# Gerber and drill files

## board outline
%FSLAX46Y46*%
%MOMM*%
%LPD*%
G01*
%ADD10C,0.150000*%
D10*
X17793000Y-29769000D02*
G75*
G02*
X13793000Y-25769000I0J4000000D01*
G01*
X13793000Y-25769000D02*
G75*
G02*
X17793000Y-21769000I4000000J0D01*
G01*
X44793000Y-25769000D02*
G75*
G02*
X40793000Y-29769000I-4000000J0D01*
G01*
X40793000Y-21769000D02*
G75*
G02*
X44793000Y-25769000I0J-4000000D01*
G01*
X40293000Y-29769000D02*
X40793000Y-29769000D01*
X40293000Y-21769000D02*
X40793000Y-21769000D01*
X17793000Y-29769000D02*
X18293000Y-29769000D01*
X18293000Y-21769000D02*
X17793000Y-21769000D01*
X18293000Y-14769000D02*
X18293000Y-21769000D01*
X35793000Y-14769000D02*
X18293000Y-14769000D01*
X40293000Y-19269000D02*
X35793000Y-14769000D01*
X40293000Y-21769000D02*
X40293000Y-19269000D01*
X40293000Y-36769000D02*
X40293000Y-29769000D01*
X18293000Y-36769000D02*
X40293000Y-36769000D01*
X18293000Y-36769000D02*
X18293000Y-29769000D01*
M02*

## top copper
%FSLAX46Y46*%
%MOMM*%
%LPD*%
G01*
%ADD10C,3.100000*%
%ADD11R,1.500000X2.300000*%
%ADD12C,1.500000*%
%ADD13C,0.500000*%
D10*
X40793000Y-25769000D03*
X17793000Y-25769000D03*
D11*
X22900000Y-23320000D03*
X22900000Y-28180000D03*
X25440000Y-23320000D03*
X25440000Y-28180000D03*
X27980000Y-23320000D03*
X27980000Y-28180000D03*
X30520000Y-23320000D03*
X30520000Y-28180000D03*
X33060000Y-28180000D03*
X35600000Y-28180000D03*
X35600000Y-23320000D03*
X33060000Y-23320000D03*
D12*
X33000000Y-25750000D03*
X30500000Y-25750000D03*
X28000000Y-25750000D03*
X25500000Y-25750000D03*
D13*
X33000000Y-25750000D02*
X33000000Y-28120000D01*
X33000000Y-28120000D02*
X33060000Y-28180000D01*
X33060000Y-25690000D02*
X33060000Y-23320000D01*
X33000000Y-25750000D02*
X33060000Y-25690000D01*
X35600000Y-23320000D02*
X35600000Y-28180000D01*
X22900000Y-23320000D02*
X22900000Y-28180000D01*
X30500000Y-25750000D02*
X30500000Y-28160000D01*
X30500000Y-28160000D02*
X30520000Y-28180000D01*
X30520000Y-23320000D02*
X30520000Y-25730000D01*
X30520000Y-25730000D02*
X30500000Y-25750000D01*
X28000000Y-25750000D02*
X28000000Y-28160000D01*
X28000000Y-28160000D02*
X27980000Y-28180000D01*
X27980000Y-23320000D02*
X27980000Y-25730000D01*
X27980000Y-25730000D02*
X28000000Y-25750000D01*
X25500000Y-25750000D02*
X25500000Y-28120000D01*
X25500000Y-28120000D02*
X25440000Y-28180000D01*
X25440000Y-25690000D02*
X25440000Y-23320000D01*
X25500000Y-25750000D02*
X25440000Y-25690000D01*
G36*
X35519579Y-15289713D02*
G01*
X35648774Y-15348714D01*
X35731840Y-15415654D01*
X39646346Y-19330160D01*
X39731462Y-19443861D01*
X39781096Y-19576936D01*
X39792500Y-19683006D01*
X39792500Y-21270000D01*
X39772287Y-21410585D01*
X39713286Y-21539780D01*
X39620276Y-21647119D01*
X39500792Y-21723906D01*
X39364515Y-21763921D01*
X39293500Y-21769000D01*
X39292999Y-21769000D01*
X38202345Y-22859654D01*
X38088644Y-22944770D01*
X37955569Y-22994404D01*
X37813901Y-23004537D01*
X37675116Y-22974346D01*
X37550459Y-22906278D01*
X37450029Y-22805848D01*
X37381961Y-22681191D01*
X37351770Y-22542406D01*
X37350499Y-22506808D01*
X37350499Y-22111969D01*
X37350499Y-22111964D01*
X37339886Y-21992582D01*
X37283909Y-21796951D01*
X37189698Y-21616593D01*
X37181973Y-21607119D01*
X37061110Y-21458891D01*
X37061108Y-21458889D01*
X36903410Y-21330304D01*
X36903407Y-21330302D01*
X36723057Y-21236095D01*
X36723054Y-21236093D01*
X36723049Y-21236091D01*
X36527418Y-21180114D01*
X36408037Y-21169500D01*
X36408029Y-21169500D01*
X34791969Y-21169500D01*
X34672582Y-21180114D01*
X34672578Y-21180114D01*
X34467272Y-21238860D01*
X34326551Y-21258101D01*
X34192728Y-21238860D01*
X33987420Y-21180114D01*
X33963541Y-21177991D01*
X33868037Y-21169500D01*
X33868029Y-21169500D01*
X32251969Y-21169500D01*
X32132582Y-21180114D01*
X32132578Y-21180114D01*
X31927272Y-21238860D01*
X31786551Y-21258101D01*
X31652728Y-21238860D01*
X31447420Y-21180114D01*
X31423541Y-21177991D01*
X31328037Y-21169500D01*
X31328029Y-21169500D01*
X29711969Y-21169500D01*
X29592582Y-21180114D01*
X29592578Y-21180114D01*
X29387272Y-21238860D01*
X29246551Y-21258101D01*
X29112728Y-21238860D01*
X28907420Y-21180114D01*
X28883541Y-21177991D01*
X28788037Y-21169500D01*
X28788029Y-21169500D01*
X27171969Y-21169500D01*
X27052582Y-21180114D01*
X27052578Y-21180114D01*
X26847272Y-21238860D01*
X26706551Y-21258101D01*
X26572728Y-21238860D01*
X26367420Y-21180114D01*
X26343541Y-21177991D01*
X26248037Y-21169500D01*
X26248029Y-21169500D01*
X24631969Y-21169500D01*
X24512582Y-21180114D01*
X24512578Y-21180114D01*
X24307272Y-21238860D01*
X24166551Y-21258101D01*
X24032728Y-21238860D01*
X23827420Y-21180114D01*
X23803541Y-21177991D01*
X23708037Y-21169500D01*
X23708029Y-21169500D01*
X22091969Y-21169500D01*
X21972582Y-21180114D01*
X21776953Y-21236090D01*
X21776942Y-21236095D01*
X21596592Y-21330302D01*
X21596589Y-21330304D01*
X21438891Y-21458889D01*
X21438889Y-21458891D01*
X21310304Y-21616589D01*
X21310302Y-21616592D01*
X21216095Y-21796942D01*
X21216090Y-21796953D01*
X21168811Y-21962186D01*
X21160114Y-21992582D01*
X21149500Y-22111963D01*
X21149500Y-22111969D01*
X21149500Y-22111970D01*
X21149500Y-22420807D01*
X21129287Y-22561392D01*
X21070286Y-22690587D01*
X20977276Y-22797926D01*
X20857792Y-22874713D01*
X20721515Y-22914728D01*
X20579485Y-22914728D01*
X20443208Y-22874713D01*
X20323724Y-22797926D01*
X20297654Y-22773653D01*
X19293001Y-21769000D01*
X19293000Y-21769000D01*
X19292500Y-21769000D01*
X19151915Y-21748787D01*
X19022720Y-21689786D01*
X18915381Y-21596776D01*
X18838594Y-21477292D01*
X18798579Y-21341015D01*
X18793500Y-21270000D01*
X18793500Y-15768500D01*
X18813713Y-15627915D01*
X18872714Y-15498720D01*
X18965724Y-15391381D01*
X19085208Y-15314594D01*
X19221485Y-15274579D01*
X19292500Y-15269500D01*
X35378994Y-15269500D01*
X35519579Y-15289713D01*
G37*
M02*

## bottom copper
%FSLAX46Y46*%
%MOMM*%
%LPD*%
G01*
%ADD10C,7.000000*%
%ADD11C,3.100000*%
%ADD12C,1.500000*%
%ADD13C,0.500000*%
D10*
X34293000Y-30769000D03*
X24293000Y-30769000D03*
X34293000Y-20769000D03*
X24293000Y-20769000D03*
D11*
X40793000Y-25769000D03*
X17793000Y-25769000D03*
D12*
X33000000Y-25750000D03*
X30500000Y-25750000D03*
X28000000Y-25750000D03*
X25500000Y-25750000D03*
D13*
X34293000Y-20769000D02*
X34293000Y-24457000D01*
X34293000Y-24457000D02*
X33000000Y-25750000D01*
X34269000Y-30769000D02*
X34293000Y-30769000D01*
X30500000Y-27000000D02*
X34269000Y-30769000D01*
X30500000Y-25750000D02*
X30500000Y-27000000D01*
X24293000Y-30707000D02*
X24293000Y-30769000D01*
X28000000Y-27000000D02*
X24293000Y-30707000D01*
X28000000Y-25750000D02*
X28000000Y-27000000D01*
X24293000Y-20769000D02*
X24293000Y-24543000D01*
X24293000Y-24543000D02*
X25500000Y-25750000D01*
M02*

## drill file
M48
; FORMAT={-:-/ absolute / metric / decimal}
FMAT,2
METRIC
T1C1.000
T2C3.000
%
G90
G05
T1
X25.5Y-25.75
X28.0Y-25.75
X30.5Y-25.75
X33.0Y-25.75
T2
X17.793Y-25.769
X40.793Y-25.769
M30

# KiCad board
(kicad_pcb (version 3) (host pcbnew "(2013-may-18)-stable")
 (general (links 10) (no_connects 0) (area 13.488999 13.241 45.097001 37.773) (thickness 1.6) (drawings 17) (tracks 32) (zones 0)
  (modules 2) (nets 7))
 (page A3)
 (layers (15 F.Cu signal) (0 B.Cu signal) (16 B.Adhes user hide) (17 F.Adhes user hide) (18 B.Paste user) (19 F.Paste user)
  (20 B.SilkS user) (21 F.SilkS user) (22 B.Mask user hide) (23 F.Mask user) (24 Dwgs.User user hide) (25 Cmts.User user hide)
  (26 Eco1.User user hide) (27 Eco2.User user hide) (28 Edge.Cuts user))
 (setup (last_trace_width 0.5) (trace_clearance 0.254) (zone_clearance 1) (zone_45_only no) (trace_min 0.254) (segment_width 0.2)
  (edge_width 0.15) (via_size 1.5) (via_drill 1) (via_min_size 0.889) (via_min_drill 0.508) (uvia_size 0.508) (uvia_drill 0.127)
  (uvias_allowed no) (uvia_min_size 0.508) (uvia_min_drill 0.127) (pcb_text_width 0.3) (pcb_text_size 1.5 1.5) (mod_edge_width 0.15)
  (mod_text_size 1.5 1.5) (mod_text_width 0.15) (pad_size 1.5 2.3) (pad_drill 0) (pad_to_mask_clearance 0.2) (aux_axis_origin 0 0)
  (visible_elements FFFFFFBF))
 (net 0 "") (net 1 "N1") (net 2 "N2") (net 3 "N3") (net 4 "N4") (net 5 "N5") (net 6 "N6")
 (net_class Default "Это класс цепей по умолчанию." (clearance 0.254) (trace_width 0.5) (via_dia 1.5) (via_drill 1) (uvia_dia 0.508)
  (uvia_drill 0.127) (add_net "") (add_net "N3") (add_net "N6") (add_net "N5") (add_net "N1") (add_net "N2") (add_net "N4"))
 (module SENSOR (layer B.Cu) (at 40.793 37.269 180)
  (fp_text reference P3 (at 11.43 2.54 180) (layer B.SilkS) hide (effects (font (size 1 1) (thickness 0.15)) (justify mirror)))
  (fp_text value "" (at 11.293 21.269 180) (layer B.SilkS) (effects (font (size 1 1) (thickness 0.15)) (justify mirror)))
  (pad 2 smd circle (at 6.5 6.5 180) (size 7 7) (layers B.Cu B.Mask) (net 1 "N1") (solder_mask_margin 0.1))
  (pad 3 smd circle (at 16.5 6.5 180) (size 7 7) (layers B.Cu B.Mask) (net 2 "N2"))
  (pad 1 smd circle (at 6.5 16.5 180) (size 7 7) (layers B.Cu B.Mask) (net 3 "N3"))
  (pad 4 smd circle (at 16.5 16.5 180) (size 7 7) (layers B.Cu B.Mask) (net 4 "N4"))
  (pad "" np_thru_hole circle (at 0 11.5 180) (size 3.1 3.1) (drill 3) (layers *.Cu *.Mask B.SilkS))
  (pad "" np_thru_hole circle (at 23 11.5 180) (size 3.1 3.1) (drill 3) (layers *.Cu *.Mask B.SilkS)))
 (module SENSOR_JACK (layer F.Cu) (at 29.25 25.75)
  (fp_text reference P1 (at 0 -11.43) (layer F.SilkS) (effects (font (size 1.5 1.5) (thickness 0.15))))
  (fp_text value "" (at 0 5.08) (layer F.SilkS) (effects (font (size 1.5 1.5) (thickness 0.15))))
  (pad 12 smd rect (at -6.35 -2.43) (size 1.5 2.3) (layers F.Cu F.Paste F.Mask) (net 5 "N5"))
  (pad 1 smd rect (at -6.35 2.43) (size 1.5 2.3) (layers F.Cu F.Paste F.Mask) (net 5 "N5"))
  (pad 11 smd rect (at -3.81 -2.43) (size 1.5 2.3) (layers F.Cu F.Paste F.Mask) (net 4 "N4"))
  (pad 2 smd rect (at -3.81 2.43) (size 1.5 2.3) (layers F.Cu F.Paste F.Mask) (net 4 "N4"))
  (pad 10 smd rect (at -1.27 -2.43) (size 1.5 2.3) (layers F.Cu F.Paste F.Mask) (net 2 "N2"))
  (pad 3 smd rect (at -1.27 2.43) (size 1.5 2.3) (layers F.Cu F.Paste F.Mask) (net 2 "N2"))
  (pad 9 smd rect (at 1.27 -2.43) (size 1.5 2.3) (layers F.Cu F.Paste F.Mask) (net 1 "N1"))
  (pad 4 smd rect (at 1.27 2.43) (size 1.5 2.3) (layers F.Cu F.Paste F.Mask) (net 1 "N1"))
  (pad 5 smd rect (at 3.81 2.43) (size 1.5 2.3) (layers F.Cu F.Paste F.Mask) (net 3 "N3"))
  (pad 6 smd rect (at 6.35 2.43) (size 1.5 2.3) (layers F.Cu F.Paste F.Mask) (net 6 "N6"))
  (pad 7 smd rect (at 6.35 -2.43) (size 1.5 2.3) (layers F.Cu F.Paste F.Mask) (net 6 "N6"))
  (pad 8 smd rect (at 3.81 -2.43) (size 1.5 2.3) (layers F.Cu F.Paste F.Mask) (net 3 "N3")))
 (gr_arc (start 17.793 25.769) (end 17.793 29.769) (angle 90) (layer Edge.Cuts) (width 0.15))
 (gr_arc (start 17.793 25.769) (end 13.793 25.769) (angle 90) (layer Edge.Cuts) (width 0.15))
 (gr_arc (start 40.793 25.769) (end 44.793 25.769) (angle 90) (layer Edge.Cuts) (width 0.15))
 (gr_arc (start 40.793 25.769) (end 40.793 21.769) (angle 90) (layer Edge.Cuts) (width 0.15))
 (gr_line (start 40.293 29.769) (end 40.793 29.769) (angle 90) (layer Edge.Cuts) (width 0.15))
 (gr_line (start 40.293 21.769) (end 40.793 21.769) (angle 90) (layer Edge.Cuts) (width 0.15))
 (gr_line (start 17.793 29.769) (end 18.293 29.769) (angle 90) (layer Edge.Cuts) (width 0.15))
 (gr_line (start 18.293 21.769) (end 17.793 21.769) (angle 90) (layer Edge.Cuts) (width 0.15))
 (gr_line (start 18.293 14.769) (end 18.293 21.769) (angle 90) (layer Edge.Cuts) (width 0.15))
 (gr_line (start 35.793 14.769) (end 18.293 14.769) (angle 90) (layer Edge.Cuts) (width 0.15))
 (gr_line (start 40.293 19.269) (end 35.793 14.769) (angle 90) (layer Edge.Cuts) (width 0.15))
 (gr_line (start 40.293 21.769) (end 40.293 19.269) (angle 90) (layer Edge.Cuts) (width 0.15))
 (gr_line (start 40.293 36.769) (end 40.293 29.769) (angle 90) (layer Edge.Cuts) (width 0.15))
 (gr_line (start 18.293 36.769) (end 40.293 36.769) (angle 90) (layer Edge.Cuts) (width 0.15))
 (gr_line (start 18.293 36.769) (end 18.293 29.769) (angle 90) (layer Edge.Cuts) (width 0.15))
 (segment (start 33 25.75) (end 33 28.12) (width 0.5) (layer F.Cu) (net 3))
 (segment (start 33 28.12) (end 33.06 28.18) (width 0.5) (layer F.Cu) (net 3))
 (segment (start 34.293 20.769) (end 34.293 24.457) (width 0.5) (layer B.Cu) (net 3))
 (segment (start 33.06 25.69) (end 33.06 23.32) (width 0.5) (layer F.Cu) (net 3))
 (segment (start 33 25.75) (end 33.06 25.69) (width 0.5) (layer F.Cu) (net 3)) (via (at 33 25.75) (size 1.5) (layers F.Cu B.Cu) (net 3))
 (segment (start 34.293 24.457) (end 33 25.75) (width 0.5) (layer B.Cu) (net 3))
 (segment (start 35.6 23.32) (end 35.6 28.18) (width 0.5) (layer F.Cu) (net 6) (status C00000))
 (segment (start 22.9 23.32) (end 22.9 28.18) (width 0.5) (layer F.Cu) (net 5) (status C00000))
 (segment (start 30.5 25.75) (end 30.5 28.16) (width 0.5) (layer F.Cu) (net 1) (status 800000))
 (segment (start 30.5 28.16) (end 30.52 28.18) (width 0.5) (layer F.Cu) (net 1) (status C00000))
 (segment (start 30.52 23.32) (end 30.52 25.73) (width 0.5) (layer F.Cu) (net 1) (status 400000))
 (segment (start 34.269 30.769) (end 34.293 30.769) (width 0.5) (layer B.Cu) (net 1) (status C00000))
 (segment (start 30.5 27) (end 34.269 30.769) (width 0.5) (layer B.Cu) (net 1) (status 800000))
 (segment (start 30.5 25.75) (end 30.5 27) (width 0.5) (layer B.Cu) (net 1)) (via (at 30.5 25.75) (size 1.5) (layers F.Cu B.Cu) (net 1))
 (segment (start 30.52 25.73) (end 30.5 25.75) (width 0.5) (layer F.Cu) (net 1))
 (segment (start 28 25.75) (end 28 28.16) (width 0.5) (layer F.Cu) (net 2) (status 800000))
 (segment (start 28 28.16) (end 27.98 28.18) (width 0.5) (layer F.Cu) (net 2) (status C00000))
 (segment (start 27.98 23.32) (end 27.98 25.73) (width 0.5) (layer F.Cu) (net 2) (status 400000))
 (segment (start 24.293 30.707) (end 24.293 30.769) (width 0.5) (layer B.Cu) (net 2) (status C00000))
 (segment (start 28 27) (end 24.293 30.707) (width 0.5) (layer B.Cu) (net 2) (status 800000))
 (segment (start 28 25.75) (end 28 27) (width 0.5) (layer B.Cu) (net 2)) (via (at 28 25.75) (size 1.5) (layers F.Cu B.Cu) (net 2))
 (segment (start 27.98 25.73) (end 28 25.75) (width 0.5) (layer F.Cu) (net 2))
 (segment (start 25.5 25.75) (end 25.5 28.12) (width 0.5) (layer F.Cu) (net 4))
 (segment (start 25.5 28.12) (end 25.44 28.18) (width 0.5) (layer F.Cu) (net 4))
 (segment (start 24.293 20.769) (end 24.293 24.543) (width 0.5) (layer B.Cu) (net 4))
 (segment (start 25.44 25.69) (end 25.44 23.32) (width 0.5) (layer F.Cu) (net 4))
 (segment (start 25.5 25.75) (end 25.44 25.69) (width 0.5) (layer F.Cu) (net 4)) (via (at 25.5 25.75) (size 1.5) (layers F.Cu B.Cu) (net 4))
 (segment (start 24.293 24.543) (end 25.5 25.75) (width 0.5) (layer B.Cu) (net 4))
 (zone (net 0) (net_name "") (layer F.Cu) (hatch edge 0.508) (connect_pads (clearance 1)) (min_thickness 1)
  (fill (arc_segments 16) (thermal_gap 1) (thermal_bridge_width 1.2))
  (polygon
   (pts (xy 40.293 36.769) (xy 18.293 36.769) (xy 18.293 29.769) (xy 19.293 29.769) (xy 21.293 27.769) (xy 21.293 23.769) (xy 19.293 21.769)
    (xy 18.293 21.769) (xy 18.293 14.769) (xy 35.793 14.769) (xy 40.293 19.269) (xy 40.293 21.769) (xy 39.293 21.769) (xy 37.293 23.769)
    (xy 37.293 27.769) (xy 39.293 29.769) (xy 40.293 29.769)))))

